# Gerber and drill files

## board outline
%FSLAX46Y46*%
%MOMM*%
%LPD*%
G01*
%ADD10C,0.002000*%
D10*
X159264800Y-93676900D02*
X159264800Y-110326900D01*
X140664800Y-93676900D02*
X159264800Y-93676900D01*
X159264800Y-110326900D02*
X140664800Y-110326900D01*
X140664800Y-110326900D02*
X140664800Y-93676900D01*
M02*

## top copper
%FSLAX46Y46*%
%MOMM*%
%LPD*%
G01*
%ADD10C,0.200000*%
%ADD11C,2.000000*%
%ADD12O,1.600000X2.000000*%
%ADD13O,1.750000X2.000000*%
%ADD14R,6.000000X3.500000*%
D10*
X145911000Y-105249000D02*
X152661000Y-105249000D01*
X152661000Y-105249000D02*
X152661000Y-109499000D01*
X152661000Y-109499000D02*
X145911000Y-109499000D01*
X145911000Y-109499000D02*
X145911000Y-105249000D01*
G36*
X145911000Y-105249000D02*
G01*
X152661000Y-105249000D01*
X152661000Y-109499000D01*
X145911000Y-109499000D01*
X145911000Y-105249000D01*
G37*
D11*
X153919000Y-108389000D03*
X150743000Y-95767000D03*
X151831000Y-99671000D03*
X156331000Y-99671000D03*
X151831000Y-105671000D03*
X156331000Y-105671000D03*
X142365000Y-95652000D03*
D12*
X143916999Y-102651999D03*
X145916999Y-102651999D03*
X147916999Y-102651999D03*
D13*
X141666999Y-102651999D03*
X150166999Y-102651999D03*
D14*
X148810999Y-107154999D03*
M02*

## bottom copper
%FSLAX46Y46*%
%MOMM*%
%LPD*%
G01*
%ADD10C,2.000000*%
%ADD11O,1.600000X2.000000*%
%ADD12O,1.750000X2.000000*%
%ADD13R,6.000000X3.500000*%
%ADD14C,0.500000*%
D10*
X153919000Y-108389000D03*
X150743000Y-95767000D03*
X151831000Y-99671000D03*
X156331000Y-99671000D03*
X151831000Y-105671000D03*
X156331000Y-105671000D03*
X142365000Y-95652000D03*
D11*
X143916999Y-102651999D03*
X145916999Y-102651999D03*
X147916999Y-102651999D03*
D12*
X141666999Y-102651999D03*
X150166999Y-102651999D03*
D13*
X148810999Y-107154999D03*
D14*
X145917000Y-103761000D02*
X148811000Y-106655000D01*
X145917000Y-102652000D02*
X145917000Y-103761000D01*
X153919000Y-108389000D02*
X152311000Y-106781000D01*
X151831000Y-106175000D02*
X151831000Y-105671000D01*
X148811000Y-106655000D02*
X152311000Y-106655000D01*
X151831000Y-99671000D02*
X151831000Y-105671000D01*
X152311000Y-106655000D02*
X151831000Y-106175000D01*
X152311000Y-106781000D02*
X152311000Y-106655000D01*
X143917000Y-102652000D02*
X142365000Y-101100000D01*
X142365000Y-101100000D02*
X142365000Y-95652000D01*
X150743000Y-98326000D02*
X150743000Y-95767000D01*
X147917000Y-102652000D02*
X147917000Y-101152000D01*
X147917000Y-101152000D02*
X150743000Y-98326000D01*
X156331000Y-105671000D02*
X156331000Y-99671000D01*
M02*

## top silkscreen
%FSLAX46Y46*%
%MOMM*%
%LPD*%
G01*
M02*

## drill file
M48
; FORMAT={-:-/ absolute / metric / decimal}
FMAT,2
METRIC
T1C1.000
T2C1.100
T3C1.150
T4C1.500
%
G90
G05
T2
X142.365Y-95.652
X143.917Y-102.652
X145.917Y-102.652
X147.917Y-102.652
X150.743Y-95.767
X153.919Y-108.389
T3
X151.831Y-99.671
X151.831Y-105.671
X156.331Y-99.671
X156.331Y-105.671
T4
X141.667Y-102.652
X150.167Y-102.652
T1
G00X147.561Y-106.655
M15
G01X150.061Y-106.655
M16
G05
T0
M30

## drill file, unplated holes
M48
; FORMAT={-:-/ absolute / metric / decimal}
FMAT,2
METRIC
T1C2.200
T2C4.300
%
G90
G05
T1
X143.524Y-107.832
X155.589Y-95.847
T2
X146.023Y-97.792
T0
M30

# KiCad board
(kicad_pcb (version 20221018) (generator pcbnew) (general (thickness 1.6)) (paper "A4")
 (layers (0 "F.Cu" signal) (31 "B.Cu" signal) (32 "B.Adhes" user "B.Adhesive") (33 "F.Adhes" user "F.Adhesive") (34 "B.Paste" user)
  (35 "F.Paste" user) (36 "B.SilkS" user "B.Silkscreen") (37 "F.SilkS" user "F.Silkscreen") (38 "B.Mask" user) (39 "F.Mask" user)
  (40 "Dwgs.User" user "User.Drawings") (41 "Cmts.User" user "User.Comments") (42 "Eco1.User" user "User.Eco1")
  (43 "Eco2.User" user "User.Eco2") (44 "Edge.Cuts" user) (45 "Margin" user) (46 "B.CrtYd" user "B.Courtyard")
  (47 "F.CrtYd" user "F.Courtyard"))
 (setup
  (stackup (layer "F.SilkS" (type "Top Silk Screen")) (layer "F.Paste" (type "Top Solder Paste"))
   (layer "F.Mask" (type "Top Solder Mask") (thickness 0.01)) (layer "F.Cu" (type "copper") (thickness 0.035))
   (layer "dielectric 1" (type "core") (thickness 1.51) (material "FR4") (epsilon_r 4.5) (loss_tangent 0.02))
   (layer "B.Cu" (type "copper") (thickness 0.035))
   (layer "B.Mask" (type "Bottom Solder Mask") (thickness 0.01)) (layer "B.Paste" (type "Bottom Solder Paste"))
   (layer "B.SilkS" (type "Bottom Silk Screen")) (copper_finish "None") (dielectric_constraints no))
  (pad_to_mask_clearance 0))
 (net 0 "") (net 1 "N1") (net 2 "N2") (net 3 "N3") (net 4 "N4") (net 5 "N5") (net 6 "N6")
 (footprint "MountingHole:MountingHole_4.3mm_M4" (layer "F.Cu") (at 146.0226 97.7919)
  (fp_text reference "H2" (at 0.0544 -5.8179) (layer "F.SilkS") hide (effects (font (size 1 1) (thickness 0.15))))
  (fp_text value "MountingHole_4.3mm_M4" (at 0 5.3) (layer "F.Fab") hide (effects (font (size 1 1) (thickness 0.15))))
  (pad "" np_thru_hole circle (at 0 0) (size 4.3 4.3) (drill 4.3) (layers "*.Cu" "*.Mask")))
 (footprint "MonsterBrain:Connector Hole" (layer "F.Cu") (at 153.919 108.389)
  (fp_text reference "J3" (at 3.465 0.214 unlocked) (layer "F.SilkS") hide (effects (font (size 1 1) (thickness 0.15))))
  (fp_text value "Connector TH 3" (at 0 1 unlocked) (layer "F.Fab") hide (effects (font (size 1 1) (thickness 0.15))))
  (pad "1" thru_hole circle (at 0 0) (size 2 2) (drill 1.1) (layers "*.Cu" "*.Mask") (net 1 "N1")))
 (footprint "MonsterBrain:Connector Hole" (layer "F.Cu") (at 150.743 95.767)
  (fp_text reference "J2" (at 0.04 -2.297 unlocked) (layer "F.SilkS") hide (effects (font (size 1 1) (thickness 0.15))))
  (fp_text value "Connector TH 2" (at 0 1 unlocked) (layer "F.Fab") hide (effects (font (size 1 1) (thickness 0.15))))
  (pad "1" thru_hole circle (at 0 0) (size 2 2) (drill 1.1) (layers "*.Cu" "*.Mask") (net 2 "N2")))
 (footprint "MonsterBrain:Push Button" (layer "F.Cu") (at 154.081 102.671)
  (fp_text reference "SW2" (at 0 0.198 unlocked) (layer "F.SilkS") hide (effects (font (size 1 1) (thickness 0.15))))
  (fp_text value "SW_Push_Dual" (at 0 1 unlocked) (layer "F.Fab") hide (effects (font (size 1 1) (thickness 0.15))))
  (pad "1" thru_hole circle (at -2.25 -3) (size 2 2) (drill 1.15) (layers "*.Cu" "*.Mask") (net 1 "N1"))
  (pad "2" thru_hole circle (at 2.25 -3) (size 2 2) (drill 1.15) (layers "*.Cu" "*.Mask") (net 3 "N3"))
  (pad "3" thru_hole circle (at -2.25 3) (size 2 2) (drill 1.15) (layers "*.Cu" "*.Mask") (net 1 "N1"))
  (pad "4" thru_hole circle (at 2.25 3) (size 2 2) (drill 1.15) (layers "*.Cu" "*.Mask") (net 3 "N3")))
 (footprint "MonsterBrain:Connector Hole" (layer "F.Cu") (at 142.365 95.652)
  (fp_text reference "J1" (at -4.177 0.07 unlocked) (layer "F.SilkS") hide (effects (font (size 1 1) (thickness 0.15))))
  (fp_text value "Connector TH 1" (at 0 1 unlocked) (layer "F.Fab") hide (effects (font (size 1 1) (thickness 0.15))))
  (pad "1" thru_hole circle (at 0 0) (size 2 2) (drill 1.1) (layers "*.Cu" "*.Mask") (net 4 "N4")))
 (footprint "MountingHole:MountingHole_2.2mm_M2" (layer "F.Cu") (at 155.589 95.847)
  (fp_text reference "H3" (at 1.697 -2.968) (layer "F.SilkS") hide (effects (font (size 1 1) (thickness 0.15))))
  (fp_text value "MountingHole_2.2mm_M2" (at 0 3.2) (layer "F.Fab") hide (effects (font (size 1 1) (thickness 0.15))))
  (pad "" np_thru_hole circle (at 0 0) (size 2.2 2.2) (drill 2.2) (layers "*.Cu" "*.Mask")))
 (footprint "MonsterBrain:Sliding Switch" (layer "F.Cu") (at 145.917 102.652)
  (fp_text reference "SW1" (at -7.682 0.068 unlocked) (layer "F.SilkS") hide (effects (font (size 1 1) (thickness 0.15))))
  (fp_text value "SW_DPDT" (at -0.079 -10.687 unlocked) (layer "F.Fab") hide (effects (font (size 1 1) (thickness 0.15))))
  (pad "1" thru_hole oval (at -2 0) (size 1.6 2) (drill 1.1) (layers "*.Cu" "*.Mask") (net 4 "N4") (thermal_bridge_angle 45))
  (pad "2" thru_hole oval (at 0 0) (size 1.6 2) (drill 1.1) (layers "*.Cu" "*.Mask") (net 1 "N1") (thermal_bridge_angle 45))
  (pad "3" thru_hole oval (at 2 0) (size 1.6 2) (drill 1.1) (layers "*.Cu" "*.Mask") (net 2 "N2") (thermal_bridge_angle 45))
  (pad "4" thru_hole oval (at -4.25 0) (size 1.75 2) (drill 1.5) (layers "*.Cu" "*.Mask") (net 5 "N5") (thermal_bridge_angle 45))
  (pad "5" thru_hole oval (at 4.25 0) (size 1.75 2) (drill 1.5) (layers "*.Cu" "*.Mask") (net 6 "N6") (thermal_bridge_angle 45)))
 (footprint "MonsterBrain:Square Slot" (layer "F.Cu") (at 149.286 107.374)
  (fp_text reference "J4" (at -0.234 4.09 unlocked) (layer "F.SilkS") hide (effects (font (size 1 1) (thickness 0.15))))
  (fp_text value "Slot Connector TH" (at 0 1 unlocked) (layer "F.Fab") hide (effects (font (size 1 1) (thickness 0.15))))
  (fp_rect (start -3.375 -2.125) (end 3.375 2.125) (stroke (width 0.2) (type solid)) (fill solid) (layer "F.Cu"))
  (pad "1" thru_hole rect (at -0.475 -0.719) (size 6 3.5) (drill oval 3.5 1 (offset 0 0.5)) (layers "*.Cu" "*.Mask") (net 1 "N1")
   (thermal_bridge_angle 45)))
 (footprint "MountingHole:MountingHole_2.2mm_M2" (layer "F.Cu") (at 143.524 107.832)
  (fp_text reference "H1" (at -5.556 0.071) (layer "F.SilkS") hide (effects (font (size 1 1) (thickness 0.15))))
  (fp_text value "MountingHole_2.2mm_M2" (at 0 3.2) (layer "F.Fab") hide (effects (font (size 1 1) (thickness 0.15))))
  (pad "" np_thru_hole circle (at 0 0) (size 2.2 2.2) (drill 2.2) (layers "*.Cu" "*.Mask")))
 (gr_line (start 159.2648 93.6769) (end 159.2648 110.3269) (stroke (width 0.002) (type solid)) (layer "Edge.Cuts"))
 (gr_line (start 140.6648 93.6769) (end 159.2648 93.6769) (stroke (width 0.002) (type solid)) (layer "Edge.Cuts"))
 (gr_line (start 159.2648 110.3269) (end 140.6648 110.3269) (stroke (width 0.002) (type solid)) (layer "Edge.Cuts"))
 (gr_line (start 140.6648 110.3269) (end 140.6648 93.6769) (stroke (width 0.002) (type solid)) (layer "Edge.Cuts"))
 (segment (start 153.919 108.389) (end 152.311 106.781) (width 0.5) (layer "B.Cu") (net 1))
 (segment (start 151.831 106.175) (end 151.831 105.671) (width 0.5) (layer "B.Cu") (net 1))
 (segment (start 148.811 106.655) (end 152.311 106.655) (width 0.5) (layer "B.Cu") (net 1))
 (segment (start 151.831 99.671) (end 151.831 105.671) (width 0.5) (layer "B.Cu") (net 1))
 (segment (start 152.311 106.655) (end 151.831 106.175) (width 0.5) (layer "B.Cu") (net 1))
 (segment (start 145.917 102.652) (end 145.917 103.761) (width 0.5) (layer "B.Cu") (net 1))
 (segment (start 152.311 106.781) (end 152.311 106.655) (width 0.5) (layer "B.Cu") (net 1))
 (segment (start 145.917 103.761) (end 148.811 106.655) (width 0.5) (layer "B.Cu") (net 1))
 (segment (start 143.917 102.652) (end 142.365 101.1) (width 0.5) (layer "B.Cu") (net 4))
 (segment (start 142.365 101.1) (end 142.365 95.652) (width 0.5) (layer "B.Cu") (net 4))
 (segment (start 150.743 98.326) (end 150.743 95.767) (width 0.5) (layer "B.Cu") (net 2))
 (segment (start 147.917 102.652) (end 147.917 101.152) (width 0.5) (layer "B.Cu") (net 2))
 (segment (start 147.917 101.152) (end 150.743 98.326) (width 0.5) (layer "B.Cu") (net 2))
 (segment (start 156.331 105.671) (end 156.331 99.671) (width 0.5) (layer "B.Cu") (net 3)))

